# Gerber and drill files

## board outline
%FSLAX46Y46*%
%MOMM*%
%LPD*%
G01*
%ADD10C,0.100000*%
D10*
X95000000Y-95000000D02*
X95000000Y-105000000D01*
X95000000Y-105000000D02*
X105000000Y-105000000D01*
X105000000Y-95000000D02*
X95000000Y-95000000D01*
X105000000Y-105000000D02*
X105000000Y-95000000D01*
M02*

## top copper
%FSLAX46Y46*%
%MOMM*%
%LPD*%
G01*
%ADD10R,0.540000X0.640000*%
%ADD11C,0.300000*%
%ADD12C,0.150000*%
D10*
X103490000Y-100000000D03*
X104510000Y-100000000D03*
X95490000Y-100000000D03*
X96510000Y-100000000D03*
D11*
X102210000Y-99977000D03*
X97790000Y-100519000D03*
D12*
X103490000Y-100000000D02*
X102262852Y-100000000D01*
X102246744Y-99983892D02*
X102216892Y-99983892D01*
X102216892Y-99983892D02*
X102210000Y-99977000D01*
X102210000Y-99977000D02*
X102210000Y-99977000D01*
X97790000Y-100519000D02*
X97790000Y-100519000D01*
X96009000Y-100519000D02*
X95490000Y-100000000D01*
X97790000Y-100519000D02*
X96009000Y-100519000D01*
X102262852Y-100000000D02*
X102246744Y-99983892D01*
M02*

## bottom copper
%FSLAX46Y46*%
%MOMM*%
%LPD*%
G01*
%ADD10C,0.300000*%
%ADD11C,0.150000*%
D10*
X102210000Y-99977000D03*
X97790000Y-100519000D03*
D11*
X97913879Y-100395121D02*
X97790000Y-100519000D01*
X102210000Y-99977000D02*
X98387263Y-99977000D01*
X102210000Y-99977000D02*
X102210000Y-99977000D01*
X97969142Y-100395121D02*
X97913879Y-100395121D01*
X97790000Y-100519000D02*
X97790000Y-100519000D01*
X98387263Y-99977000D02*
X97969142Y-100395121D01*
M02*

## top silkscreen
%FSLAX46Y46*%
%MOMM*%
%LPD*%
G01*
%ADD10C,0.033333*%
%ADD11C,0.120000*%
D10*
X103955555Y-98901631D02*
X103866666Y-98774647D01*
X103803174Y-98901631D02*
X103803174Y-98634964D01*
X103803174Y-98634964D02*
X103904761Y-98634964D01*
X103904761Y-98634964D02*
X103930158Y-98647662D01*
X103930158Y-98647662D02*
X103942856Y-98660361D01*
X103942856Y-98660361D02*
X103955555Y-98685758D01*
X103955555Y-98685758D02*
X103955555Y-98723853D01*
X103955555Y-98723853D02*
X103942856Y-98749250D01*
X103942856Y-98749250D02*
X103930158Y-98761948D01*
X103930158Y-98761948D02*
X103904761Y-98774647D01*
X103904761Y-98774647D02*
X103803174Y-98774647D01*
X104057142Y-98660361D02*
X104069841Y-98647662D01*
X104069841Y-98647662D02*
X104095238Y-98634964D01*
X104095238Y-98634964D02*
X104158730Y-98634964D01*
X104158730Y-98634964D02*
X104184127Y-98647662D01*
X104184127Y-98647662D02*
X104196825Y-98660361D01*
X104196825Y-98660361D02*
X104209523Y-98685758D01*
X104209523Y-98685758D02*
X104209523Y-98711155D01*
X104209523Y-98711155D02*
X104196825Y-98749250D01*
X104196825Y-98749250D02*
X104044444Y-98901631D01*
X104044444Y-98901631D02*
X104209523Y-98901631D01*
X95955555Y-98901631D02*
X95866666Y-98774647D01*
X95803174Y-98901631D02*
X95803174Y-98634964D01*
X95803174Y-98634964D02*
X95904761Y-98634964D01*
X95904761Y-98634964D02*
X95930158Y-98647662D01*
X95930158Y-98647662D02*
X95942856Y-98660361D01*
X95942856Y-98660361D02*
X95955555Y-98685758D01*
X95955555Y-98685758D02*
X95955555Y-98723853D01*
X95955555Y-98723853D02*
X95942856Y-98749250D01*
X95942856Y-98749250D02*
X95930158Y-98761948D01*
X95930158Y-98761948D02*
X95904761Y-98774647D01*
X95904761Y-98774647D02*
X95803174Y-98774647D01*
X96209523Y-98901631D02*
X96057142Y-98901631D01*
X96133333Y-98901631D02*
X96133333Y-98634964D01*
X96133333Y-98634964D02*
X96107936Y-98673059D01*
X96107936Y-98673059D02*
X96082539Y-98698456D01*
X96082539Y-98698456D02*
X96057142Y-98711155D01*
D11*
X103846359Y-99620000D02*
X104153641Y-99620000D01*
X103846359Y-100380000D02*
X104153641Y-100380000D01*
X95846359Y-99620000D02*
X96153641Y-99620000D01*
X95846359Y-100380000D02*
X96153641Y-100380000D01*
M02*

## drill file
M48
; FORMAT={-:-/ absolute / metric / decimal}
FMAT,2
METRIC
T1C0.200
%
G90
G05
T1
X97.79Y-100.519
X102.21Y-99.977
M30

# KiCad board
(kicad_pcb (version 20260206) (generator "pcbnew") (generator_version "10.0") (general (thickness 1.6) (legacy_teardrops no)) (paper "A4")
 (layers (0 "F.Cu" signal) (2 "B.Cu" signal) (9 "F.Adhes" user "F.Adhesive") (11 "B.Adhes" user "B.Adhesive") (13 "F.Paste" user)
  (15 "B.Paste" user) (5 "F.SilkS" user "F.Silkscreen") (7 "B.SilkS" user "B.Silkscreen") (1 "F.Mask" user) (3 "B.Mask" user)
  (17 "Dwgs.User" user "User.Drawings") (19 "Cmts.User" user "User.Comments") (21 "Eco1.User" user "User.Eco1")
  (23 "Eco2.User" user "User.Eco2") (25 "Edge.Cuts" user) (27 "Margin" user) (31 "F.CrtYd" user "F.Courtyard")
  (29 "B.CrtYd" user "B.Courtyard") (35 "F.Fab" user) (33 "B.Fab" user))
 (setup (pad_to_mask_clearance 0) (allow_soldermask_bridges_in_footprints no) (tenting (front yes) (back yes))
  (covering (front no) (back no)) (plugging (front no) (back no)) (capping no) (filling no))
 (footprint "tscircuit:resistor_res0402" (layer "F.Cu") (at 104 100)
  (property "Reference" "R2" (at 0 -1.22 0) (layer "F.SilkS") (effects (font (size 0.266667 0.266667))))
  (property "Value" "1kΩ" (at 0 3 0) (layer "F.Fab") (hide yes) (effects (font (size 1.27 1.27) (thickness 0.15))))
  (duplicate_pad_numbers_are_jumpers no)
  (fp_line (start -0.153641 -0.38) (end 0.153641 -0.38) (stroke (width 0.12) (type default)) (layer "F.SilkS"))
  (fp_line (start -0.153641 0.38) (end 0.153641 0.38) (stroke (width 0.12) (type default)) (layer "F.SilkS"))
  (pad "1" smd rect (at -0.51 0) (size 0.54 0.64) (layers "F.Cu" "F.Mask" "F.Paste") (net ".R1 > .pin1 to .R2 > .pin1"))
  (pad "2" smd rect (at 0.51 0) (size 0.54 0.64) (layers "F.Cu" "F.Mask" "F.Paste")))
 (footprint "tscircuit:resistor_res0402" (layer "F.Cu") (at 96 100)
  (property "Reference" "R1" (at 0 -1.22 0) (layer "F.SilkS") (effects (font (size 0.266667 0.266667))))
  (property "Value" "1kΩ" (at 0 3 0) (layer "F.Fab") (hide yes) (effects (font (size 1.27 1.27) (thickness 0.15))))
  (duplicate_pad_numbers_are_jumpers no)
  (fp_line (start -0.153641 -0.38) (end 0.153641 -0.38) (stroke (width 0.12) (type default)) (layer "F.SilkS"))
  (fp_line (start -0.153641 0.38) (end 0.153641 0.38) (stroke (width 0.12) (type default)) (layer "F.SilkS"))
  (pad "1" smd rect (at -0.51 0) (size 0.54 0.64) (layers "F.Cu" "F.Mask" "F.Paste") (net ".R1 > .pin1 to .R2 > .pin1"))
  (pad "2" smd rect (at 0.51 0) (size 0.54 0.64) (layers "F.Cu" "F.Mask" "F.Paste")))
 (gr_line (start 95 95) (end 95 105) (stroke (width 0.1) (type solid)) (layer "Edge.Cuts"))
 (gr_line (start 95 105) (end 105 105) (stroke (width 0.1) (type solid)) (layer "Edge.Cuts"))
 (gr_line (start 105 95) (end 95 95) (stroke (width 0.1) (type solid)) (layer "Edge.Cuts"))
 (gr_line (start 105 105) (end 105 95) (stroke (width 0.1) (type solid)) (layer "Edge.Cuts"))
 (segment (start 103.49 100) (end 102.262852 100) (width 0.15) (layer "F.Cu") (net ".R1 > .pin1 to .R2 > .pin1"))
 (segment (start 102.246744 99.983892) (end 102.216892 99.983892) (width 0.15) (layer "F.Cu") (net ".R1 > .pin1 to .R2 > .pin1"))
 (segment (start 102.216892 99.983892) (end 102.21 99.977) (width 0.15) (layer "F.Cu") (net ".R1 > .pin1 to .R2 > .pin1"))
 (segment (start 102.21 99.977) (end 102.21 99.977) (width 0.15) (layer "F.Cu") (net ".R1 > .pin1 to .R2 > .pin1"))
 (segment (start 97.79 100.519) (end 97.79 100.519) (width 0.15) (layer "F.Cu") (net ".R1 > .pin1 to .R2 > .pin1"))
 (segment (start 96.009 100.519) (end 95.49 100) (width 0.15) (layer "F.Cu") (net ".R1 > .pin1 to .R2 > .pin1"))
 (segment (start 97.79 100.519) (end 96.009 100.519) (width 0.15) (layer "F.Cu") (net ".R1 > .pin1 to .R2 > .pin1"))
 (segment (start 102.262852 100) (end 102.246744 99.983892) (width 0.15) (layer "F.Cu") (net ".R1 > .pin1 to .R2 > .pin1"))
 (via (at 102.21 99.977) (size 0.3) (drill 0.2) (layers "F.Cu" "B.Cu") (capping no) (covering (front no) (back no))
  (plugging (front no) (back no)) (filling no) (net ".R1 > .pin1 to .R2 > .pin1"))
 (via (at 97.79 100.519) (size 0.3) (drill 0.2) (layers "F.Cu" "B.Cu") (capping no) (covering (front no) (back no))
  (plugging (front no) (back no)) (filling no) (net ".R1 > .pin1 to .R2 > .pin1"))
 (segment (start 97.913879 100.395121) (end 97.79 100.519) (width 0.15) (layer "B.Cu") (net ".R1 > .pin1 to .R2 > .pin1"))
 (segment (start 102.21 99.977) (end 98.387263 99.977) (width 0.15) (layer "B.Cu") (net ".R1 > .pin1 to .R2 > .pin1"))
 (segment (start 102.21 99.977) (end 102.21 99.977) (width 0.15) (layer "B.Cu") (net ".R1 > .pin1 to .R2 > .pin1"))
 (segment (start 97.969142 100.395121) (end 97.913879 100.395121) (width 0.15) (layer "B.Cu") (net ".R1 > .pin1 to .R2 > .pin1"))
 (segment (start 97.79 100.519) (end 97.79 100.519) (width 0.15) (layer "B.Cu") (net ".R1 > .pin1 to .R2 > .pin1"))
 (segment (start 98.387263 99.977) (end 97.969142 100.395121) (width 0.15) (layer "B.Cu") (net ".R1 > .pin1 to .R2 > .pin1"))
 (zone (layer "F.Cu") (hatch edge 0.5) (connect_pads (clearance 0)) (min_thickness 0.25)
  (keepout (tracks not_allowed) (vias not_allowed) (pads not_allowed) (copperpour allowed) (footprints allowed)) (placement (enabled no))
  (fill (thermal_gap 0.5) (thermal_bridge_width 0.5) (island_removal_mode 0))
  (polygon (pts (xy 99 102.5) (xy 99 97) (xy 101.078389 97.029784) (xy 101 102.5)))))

